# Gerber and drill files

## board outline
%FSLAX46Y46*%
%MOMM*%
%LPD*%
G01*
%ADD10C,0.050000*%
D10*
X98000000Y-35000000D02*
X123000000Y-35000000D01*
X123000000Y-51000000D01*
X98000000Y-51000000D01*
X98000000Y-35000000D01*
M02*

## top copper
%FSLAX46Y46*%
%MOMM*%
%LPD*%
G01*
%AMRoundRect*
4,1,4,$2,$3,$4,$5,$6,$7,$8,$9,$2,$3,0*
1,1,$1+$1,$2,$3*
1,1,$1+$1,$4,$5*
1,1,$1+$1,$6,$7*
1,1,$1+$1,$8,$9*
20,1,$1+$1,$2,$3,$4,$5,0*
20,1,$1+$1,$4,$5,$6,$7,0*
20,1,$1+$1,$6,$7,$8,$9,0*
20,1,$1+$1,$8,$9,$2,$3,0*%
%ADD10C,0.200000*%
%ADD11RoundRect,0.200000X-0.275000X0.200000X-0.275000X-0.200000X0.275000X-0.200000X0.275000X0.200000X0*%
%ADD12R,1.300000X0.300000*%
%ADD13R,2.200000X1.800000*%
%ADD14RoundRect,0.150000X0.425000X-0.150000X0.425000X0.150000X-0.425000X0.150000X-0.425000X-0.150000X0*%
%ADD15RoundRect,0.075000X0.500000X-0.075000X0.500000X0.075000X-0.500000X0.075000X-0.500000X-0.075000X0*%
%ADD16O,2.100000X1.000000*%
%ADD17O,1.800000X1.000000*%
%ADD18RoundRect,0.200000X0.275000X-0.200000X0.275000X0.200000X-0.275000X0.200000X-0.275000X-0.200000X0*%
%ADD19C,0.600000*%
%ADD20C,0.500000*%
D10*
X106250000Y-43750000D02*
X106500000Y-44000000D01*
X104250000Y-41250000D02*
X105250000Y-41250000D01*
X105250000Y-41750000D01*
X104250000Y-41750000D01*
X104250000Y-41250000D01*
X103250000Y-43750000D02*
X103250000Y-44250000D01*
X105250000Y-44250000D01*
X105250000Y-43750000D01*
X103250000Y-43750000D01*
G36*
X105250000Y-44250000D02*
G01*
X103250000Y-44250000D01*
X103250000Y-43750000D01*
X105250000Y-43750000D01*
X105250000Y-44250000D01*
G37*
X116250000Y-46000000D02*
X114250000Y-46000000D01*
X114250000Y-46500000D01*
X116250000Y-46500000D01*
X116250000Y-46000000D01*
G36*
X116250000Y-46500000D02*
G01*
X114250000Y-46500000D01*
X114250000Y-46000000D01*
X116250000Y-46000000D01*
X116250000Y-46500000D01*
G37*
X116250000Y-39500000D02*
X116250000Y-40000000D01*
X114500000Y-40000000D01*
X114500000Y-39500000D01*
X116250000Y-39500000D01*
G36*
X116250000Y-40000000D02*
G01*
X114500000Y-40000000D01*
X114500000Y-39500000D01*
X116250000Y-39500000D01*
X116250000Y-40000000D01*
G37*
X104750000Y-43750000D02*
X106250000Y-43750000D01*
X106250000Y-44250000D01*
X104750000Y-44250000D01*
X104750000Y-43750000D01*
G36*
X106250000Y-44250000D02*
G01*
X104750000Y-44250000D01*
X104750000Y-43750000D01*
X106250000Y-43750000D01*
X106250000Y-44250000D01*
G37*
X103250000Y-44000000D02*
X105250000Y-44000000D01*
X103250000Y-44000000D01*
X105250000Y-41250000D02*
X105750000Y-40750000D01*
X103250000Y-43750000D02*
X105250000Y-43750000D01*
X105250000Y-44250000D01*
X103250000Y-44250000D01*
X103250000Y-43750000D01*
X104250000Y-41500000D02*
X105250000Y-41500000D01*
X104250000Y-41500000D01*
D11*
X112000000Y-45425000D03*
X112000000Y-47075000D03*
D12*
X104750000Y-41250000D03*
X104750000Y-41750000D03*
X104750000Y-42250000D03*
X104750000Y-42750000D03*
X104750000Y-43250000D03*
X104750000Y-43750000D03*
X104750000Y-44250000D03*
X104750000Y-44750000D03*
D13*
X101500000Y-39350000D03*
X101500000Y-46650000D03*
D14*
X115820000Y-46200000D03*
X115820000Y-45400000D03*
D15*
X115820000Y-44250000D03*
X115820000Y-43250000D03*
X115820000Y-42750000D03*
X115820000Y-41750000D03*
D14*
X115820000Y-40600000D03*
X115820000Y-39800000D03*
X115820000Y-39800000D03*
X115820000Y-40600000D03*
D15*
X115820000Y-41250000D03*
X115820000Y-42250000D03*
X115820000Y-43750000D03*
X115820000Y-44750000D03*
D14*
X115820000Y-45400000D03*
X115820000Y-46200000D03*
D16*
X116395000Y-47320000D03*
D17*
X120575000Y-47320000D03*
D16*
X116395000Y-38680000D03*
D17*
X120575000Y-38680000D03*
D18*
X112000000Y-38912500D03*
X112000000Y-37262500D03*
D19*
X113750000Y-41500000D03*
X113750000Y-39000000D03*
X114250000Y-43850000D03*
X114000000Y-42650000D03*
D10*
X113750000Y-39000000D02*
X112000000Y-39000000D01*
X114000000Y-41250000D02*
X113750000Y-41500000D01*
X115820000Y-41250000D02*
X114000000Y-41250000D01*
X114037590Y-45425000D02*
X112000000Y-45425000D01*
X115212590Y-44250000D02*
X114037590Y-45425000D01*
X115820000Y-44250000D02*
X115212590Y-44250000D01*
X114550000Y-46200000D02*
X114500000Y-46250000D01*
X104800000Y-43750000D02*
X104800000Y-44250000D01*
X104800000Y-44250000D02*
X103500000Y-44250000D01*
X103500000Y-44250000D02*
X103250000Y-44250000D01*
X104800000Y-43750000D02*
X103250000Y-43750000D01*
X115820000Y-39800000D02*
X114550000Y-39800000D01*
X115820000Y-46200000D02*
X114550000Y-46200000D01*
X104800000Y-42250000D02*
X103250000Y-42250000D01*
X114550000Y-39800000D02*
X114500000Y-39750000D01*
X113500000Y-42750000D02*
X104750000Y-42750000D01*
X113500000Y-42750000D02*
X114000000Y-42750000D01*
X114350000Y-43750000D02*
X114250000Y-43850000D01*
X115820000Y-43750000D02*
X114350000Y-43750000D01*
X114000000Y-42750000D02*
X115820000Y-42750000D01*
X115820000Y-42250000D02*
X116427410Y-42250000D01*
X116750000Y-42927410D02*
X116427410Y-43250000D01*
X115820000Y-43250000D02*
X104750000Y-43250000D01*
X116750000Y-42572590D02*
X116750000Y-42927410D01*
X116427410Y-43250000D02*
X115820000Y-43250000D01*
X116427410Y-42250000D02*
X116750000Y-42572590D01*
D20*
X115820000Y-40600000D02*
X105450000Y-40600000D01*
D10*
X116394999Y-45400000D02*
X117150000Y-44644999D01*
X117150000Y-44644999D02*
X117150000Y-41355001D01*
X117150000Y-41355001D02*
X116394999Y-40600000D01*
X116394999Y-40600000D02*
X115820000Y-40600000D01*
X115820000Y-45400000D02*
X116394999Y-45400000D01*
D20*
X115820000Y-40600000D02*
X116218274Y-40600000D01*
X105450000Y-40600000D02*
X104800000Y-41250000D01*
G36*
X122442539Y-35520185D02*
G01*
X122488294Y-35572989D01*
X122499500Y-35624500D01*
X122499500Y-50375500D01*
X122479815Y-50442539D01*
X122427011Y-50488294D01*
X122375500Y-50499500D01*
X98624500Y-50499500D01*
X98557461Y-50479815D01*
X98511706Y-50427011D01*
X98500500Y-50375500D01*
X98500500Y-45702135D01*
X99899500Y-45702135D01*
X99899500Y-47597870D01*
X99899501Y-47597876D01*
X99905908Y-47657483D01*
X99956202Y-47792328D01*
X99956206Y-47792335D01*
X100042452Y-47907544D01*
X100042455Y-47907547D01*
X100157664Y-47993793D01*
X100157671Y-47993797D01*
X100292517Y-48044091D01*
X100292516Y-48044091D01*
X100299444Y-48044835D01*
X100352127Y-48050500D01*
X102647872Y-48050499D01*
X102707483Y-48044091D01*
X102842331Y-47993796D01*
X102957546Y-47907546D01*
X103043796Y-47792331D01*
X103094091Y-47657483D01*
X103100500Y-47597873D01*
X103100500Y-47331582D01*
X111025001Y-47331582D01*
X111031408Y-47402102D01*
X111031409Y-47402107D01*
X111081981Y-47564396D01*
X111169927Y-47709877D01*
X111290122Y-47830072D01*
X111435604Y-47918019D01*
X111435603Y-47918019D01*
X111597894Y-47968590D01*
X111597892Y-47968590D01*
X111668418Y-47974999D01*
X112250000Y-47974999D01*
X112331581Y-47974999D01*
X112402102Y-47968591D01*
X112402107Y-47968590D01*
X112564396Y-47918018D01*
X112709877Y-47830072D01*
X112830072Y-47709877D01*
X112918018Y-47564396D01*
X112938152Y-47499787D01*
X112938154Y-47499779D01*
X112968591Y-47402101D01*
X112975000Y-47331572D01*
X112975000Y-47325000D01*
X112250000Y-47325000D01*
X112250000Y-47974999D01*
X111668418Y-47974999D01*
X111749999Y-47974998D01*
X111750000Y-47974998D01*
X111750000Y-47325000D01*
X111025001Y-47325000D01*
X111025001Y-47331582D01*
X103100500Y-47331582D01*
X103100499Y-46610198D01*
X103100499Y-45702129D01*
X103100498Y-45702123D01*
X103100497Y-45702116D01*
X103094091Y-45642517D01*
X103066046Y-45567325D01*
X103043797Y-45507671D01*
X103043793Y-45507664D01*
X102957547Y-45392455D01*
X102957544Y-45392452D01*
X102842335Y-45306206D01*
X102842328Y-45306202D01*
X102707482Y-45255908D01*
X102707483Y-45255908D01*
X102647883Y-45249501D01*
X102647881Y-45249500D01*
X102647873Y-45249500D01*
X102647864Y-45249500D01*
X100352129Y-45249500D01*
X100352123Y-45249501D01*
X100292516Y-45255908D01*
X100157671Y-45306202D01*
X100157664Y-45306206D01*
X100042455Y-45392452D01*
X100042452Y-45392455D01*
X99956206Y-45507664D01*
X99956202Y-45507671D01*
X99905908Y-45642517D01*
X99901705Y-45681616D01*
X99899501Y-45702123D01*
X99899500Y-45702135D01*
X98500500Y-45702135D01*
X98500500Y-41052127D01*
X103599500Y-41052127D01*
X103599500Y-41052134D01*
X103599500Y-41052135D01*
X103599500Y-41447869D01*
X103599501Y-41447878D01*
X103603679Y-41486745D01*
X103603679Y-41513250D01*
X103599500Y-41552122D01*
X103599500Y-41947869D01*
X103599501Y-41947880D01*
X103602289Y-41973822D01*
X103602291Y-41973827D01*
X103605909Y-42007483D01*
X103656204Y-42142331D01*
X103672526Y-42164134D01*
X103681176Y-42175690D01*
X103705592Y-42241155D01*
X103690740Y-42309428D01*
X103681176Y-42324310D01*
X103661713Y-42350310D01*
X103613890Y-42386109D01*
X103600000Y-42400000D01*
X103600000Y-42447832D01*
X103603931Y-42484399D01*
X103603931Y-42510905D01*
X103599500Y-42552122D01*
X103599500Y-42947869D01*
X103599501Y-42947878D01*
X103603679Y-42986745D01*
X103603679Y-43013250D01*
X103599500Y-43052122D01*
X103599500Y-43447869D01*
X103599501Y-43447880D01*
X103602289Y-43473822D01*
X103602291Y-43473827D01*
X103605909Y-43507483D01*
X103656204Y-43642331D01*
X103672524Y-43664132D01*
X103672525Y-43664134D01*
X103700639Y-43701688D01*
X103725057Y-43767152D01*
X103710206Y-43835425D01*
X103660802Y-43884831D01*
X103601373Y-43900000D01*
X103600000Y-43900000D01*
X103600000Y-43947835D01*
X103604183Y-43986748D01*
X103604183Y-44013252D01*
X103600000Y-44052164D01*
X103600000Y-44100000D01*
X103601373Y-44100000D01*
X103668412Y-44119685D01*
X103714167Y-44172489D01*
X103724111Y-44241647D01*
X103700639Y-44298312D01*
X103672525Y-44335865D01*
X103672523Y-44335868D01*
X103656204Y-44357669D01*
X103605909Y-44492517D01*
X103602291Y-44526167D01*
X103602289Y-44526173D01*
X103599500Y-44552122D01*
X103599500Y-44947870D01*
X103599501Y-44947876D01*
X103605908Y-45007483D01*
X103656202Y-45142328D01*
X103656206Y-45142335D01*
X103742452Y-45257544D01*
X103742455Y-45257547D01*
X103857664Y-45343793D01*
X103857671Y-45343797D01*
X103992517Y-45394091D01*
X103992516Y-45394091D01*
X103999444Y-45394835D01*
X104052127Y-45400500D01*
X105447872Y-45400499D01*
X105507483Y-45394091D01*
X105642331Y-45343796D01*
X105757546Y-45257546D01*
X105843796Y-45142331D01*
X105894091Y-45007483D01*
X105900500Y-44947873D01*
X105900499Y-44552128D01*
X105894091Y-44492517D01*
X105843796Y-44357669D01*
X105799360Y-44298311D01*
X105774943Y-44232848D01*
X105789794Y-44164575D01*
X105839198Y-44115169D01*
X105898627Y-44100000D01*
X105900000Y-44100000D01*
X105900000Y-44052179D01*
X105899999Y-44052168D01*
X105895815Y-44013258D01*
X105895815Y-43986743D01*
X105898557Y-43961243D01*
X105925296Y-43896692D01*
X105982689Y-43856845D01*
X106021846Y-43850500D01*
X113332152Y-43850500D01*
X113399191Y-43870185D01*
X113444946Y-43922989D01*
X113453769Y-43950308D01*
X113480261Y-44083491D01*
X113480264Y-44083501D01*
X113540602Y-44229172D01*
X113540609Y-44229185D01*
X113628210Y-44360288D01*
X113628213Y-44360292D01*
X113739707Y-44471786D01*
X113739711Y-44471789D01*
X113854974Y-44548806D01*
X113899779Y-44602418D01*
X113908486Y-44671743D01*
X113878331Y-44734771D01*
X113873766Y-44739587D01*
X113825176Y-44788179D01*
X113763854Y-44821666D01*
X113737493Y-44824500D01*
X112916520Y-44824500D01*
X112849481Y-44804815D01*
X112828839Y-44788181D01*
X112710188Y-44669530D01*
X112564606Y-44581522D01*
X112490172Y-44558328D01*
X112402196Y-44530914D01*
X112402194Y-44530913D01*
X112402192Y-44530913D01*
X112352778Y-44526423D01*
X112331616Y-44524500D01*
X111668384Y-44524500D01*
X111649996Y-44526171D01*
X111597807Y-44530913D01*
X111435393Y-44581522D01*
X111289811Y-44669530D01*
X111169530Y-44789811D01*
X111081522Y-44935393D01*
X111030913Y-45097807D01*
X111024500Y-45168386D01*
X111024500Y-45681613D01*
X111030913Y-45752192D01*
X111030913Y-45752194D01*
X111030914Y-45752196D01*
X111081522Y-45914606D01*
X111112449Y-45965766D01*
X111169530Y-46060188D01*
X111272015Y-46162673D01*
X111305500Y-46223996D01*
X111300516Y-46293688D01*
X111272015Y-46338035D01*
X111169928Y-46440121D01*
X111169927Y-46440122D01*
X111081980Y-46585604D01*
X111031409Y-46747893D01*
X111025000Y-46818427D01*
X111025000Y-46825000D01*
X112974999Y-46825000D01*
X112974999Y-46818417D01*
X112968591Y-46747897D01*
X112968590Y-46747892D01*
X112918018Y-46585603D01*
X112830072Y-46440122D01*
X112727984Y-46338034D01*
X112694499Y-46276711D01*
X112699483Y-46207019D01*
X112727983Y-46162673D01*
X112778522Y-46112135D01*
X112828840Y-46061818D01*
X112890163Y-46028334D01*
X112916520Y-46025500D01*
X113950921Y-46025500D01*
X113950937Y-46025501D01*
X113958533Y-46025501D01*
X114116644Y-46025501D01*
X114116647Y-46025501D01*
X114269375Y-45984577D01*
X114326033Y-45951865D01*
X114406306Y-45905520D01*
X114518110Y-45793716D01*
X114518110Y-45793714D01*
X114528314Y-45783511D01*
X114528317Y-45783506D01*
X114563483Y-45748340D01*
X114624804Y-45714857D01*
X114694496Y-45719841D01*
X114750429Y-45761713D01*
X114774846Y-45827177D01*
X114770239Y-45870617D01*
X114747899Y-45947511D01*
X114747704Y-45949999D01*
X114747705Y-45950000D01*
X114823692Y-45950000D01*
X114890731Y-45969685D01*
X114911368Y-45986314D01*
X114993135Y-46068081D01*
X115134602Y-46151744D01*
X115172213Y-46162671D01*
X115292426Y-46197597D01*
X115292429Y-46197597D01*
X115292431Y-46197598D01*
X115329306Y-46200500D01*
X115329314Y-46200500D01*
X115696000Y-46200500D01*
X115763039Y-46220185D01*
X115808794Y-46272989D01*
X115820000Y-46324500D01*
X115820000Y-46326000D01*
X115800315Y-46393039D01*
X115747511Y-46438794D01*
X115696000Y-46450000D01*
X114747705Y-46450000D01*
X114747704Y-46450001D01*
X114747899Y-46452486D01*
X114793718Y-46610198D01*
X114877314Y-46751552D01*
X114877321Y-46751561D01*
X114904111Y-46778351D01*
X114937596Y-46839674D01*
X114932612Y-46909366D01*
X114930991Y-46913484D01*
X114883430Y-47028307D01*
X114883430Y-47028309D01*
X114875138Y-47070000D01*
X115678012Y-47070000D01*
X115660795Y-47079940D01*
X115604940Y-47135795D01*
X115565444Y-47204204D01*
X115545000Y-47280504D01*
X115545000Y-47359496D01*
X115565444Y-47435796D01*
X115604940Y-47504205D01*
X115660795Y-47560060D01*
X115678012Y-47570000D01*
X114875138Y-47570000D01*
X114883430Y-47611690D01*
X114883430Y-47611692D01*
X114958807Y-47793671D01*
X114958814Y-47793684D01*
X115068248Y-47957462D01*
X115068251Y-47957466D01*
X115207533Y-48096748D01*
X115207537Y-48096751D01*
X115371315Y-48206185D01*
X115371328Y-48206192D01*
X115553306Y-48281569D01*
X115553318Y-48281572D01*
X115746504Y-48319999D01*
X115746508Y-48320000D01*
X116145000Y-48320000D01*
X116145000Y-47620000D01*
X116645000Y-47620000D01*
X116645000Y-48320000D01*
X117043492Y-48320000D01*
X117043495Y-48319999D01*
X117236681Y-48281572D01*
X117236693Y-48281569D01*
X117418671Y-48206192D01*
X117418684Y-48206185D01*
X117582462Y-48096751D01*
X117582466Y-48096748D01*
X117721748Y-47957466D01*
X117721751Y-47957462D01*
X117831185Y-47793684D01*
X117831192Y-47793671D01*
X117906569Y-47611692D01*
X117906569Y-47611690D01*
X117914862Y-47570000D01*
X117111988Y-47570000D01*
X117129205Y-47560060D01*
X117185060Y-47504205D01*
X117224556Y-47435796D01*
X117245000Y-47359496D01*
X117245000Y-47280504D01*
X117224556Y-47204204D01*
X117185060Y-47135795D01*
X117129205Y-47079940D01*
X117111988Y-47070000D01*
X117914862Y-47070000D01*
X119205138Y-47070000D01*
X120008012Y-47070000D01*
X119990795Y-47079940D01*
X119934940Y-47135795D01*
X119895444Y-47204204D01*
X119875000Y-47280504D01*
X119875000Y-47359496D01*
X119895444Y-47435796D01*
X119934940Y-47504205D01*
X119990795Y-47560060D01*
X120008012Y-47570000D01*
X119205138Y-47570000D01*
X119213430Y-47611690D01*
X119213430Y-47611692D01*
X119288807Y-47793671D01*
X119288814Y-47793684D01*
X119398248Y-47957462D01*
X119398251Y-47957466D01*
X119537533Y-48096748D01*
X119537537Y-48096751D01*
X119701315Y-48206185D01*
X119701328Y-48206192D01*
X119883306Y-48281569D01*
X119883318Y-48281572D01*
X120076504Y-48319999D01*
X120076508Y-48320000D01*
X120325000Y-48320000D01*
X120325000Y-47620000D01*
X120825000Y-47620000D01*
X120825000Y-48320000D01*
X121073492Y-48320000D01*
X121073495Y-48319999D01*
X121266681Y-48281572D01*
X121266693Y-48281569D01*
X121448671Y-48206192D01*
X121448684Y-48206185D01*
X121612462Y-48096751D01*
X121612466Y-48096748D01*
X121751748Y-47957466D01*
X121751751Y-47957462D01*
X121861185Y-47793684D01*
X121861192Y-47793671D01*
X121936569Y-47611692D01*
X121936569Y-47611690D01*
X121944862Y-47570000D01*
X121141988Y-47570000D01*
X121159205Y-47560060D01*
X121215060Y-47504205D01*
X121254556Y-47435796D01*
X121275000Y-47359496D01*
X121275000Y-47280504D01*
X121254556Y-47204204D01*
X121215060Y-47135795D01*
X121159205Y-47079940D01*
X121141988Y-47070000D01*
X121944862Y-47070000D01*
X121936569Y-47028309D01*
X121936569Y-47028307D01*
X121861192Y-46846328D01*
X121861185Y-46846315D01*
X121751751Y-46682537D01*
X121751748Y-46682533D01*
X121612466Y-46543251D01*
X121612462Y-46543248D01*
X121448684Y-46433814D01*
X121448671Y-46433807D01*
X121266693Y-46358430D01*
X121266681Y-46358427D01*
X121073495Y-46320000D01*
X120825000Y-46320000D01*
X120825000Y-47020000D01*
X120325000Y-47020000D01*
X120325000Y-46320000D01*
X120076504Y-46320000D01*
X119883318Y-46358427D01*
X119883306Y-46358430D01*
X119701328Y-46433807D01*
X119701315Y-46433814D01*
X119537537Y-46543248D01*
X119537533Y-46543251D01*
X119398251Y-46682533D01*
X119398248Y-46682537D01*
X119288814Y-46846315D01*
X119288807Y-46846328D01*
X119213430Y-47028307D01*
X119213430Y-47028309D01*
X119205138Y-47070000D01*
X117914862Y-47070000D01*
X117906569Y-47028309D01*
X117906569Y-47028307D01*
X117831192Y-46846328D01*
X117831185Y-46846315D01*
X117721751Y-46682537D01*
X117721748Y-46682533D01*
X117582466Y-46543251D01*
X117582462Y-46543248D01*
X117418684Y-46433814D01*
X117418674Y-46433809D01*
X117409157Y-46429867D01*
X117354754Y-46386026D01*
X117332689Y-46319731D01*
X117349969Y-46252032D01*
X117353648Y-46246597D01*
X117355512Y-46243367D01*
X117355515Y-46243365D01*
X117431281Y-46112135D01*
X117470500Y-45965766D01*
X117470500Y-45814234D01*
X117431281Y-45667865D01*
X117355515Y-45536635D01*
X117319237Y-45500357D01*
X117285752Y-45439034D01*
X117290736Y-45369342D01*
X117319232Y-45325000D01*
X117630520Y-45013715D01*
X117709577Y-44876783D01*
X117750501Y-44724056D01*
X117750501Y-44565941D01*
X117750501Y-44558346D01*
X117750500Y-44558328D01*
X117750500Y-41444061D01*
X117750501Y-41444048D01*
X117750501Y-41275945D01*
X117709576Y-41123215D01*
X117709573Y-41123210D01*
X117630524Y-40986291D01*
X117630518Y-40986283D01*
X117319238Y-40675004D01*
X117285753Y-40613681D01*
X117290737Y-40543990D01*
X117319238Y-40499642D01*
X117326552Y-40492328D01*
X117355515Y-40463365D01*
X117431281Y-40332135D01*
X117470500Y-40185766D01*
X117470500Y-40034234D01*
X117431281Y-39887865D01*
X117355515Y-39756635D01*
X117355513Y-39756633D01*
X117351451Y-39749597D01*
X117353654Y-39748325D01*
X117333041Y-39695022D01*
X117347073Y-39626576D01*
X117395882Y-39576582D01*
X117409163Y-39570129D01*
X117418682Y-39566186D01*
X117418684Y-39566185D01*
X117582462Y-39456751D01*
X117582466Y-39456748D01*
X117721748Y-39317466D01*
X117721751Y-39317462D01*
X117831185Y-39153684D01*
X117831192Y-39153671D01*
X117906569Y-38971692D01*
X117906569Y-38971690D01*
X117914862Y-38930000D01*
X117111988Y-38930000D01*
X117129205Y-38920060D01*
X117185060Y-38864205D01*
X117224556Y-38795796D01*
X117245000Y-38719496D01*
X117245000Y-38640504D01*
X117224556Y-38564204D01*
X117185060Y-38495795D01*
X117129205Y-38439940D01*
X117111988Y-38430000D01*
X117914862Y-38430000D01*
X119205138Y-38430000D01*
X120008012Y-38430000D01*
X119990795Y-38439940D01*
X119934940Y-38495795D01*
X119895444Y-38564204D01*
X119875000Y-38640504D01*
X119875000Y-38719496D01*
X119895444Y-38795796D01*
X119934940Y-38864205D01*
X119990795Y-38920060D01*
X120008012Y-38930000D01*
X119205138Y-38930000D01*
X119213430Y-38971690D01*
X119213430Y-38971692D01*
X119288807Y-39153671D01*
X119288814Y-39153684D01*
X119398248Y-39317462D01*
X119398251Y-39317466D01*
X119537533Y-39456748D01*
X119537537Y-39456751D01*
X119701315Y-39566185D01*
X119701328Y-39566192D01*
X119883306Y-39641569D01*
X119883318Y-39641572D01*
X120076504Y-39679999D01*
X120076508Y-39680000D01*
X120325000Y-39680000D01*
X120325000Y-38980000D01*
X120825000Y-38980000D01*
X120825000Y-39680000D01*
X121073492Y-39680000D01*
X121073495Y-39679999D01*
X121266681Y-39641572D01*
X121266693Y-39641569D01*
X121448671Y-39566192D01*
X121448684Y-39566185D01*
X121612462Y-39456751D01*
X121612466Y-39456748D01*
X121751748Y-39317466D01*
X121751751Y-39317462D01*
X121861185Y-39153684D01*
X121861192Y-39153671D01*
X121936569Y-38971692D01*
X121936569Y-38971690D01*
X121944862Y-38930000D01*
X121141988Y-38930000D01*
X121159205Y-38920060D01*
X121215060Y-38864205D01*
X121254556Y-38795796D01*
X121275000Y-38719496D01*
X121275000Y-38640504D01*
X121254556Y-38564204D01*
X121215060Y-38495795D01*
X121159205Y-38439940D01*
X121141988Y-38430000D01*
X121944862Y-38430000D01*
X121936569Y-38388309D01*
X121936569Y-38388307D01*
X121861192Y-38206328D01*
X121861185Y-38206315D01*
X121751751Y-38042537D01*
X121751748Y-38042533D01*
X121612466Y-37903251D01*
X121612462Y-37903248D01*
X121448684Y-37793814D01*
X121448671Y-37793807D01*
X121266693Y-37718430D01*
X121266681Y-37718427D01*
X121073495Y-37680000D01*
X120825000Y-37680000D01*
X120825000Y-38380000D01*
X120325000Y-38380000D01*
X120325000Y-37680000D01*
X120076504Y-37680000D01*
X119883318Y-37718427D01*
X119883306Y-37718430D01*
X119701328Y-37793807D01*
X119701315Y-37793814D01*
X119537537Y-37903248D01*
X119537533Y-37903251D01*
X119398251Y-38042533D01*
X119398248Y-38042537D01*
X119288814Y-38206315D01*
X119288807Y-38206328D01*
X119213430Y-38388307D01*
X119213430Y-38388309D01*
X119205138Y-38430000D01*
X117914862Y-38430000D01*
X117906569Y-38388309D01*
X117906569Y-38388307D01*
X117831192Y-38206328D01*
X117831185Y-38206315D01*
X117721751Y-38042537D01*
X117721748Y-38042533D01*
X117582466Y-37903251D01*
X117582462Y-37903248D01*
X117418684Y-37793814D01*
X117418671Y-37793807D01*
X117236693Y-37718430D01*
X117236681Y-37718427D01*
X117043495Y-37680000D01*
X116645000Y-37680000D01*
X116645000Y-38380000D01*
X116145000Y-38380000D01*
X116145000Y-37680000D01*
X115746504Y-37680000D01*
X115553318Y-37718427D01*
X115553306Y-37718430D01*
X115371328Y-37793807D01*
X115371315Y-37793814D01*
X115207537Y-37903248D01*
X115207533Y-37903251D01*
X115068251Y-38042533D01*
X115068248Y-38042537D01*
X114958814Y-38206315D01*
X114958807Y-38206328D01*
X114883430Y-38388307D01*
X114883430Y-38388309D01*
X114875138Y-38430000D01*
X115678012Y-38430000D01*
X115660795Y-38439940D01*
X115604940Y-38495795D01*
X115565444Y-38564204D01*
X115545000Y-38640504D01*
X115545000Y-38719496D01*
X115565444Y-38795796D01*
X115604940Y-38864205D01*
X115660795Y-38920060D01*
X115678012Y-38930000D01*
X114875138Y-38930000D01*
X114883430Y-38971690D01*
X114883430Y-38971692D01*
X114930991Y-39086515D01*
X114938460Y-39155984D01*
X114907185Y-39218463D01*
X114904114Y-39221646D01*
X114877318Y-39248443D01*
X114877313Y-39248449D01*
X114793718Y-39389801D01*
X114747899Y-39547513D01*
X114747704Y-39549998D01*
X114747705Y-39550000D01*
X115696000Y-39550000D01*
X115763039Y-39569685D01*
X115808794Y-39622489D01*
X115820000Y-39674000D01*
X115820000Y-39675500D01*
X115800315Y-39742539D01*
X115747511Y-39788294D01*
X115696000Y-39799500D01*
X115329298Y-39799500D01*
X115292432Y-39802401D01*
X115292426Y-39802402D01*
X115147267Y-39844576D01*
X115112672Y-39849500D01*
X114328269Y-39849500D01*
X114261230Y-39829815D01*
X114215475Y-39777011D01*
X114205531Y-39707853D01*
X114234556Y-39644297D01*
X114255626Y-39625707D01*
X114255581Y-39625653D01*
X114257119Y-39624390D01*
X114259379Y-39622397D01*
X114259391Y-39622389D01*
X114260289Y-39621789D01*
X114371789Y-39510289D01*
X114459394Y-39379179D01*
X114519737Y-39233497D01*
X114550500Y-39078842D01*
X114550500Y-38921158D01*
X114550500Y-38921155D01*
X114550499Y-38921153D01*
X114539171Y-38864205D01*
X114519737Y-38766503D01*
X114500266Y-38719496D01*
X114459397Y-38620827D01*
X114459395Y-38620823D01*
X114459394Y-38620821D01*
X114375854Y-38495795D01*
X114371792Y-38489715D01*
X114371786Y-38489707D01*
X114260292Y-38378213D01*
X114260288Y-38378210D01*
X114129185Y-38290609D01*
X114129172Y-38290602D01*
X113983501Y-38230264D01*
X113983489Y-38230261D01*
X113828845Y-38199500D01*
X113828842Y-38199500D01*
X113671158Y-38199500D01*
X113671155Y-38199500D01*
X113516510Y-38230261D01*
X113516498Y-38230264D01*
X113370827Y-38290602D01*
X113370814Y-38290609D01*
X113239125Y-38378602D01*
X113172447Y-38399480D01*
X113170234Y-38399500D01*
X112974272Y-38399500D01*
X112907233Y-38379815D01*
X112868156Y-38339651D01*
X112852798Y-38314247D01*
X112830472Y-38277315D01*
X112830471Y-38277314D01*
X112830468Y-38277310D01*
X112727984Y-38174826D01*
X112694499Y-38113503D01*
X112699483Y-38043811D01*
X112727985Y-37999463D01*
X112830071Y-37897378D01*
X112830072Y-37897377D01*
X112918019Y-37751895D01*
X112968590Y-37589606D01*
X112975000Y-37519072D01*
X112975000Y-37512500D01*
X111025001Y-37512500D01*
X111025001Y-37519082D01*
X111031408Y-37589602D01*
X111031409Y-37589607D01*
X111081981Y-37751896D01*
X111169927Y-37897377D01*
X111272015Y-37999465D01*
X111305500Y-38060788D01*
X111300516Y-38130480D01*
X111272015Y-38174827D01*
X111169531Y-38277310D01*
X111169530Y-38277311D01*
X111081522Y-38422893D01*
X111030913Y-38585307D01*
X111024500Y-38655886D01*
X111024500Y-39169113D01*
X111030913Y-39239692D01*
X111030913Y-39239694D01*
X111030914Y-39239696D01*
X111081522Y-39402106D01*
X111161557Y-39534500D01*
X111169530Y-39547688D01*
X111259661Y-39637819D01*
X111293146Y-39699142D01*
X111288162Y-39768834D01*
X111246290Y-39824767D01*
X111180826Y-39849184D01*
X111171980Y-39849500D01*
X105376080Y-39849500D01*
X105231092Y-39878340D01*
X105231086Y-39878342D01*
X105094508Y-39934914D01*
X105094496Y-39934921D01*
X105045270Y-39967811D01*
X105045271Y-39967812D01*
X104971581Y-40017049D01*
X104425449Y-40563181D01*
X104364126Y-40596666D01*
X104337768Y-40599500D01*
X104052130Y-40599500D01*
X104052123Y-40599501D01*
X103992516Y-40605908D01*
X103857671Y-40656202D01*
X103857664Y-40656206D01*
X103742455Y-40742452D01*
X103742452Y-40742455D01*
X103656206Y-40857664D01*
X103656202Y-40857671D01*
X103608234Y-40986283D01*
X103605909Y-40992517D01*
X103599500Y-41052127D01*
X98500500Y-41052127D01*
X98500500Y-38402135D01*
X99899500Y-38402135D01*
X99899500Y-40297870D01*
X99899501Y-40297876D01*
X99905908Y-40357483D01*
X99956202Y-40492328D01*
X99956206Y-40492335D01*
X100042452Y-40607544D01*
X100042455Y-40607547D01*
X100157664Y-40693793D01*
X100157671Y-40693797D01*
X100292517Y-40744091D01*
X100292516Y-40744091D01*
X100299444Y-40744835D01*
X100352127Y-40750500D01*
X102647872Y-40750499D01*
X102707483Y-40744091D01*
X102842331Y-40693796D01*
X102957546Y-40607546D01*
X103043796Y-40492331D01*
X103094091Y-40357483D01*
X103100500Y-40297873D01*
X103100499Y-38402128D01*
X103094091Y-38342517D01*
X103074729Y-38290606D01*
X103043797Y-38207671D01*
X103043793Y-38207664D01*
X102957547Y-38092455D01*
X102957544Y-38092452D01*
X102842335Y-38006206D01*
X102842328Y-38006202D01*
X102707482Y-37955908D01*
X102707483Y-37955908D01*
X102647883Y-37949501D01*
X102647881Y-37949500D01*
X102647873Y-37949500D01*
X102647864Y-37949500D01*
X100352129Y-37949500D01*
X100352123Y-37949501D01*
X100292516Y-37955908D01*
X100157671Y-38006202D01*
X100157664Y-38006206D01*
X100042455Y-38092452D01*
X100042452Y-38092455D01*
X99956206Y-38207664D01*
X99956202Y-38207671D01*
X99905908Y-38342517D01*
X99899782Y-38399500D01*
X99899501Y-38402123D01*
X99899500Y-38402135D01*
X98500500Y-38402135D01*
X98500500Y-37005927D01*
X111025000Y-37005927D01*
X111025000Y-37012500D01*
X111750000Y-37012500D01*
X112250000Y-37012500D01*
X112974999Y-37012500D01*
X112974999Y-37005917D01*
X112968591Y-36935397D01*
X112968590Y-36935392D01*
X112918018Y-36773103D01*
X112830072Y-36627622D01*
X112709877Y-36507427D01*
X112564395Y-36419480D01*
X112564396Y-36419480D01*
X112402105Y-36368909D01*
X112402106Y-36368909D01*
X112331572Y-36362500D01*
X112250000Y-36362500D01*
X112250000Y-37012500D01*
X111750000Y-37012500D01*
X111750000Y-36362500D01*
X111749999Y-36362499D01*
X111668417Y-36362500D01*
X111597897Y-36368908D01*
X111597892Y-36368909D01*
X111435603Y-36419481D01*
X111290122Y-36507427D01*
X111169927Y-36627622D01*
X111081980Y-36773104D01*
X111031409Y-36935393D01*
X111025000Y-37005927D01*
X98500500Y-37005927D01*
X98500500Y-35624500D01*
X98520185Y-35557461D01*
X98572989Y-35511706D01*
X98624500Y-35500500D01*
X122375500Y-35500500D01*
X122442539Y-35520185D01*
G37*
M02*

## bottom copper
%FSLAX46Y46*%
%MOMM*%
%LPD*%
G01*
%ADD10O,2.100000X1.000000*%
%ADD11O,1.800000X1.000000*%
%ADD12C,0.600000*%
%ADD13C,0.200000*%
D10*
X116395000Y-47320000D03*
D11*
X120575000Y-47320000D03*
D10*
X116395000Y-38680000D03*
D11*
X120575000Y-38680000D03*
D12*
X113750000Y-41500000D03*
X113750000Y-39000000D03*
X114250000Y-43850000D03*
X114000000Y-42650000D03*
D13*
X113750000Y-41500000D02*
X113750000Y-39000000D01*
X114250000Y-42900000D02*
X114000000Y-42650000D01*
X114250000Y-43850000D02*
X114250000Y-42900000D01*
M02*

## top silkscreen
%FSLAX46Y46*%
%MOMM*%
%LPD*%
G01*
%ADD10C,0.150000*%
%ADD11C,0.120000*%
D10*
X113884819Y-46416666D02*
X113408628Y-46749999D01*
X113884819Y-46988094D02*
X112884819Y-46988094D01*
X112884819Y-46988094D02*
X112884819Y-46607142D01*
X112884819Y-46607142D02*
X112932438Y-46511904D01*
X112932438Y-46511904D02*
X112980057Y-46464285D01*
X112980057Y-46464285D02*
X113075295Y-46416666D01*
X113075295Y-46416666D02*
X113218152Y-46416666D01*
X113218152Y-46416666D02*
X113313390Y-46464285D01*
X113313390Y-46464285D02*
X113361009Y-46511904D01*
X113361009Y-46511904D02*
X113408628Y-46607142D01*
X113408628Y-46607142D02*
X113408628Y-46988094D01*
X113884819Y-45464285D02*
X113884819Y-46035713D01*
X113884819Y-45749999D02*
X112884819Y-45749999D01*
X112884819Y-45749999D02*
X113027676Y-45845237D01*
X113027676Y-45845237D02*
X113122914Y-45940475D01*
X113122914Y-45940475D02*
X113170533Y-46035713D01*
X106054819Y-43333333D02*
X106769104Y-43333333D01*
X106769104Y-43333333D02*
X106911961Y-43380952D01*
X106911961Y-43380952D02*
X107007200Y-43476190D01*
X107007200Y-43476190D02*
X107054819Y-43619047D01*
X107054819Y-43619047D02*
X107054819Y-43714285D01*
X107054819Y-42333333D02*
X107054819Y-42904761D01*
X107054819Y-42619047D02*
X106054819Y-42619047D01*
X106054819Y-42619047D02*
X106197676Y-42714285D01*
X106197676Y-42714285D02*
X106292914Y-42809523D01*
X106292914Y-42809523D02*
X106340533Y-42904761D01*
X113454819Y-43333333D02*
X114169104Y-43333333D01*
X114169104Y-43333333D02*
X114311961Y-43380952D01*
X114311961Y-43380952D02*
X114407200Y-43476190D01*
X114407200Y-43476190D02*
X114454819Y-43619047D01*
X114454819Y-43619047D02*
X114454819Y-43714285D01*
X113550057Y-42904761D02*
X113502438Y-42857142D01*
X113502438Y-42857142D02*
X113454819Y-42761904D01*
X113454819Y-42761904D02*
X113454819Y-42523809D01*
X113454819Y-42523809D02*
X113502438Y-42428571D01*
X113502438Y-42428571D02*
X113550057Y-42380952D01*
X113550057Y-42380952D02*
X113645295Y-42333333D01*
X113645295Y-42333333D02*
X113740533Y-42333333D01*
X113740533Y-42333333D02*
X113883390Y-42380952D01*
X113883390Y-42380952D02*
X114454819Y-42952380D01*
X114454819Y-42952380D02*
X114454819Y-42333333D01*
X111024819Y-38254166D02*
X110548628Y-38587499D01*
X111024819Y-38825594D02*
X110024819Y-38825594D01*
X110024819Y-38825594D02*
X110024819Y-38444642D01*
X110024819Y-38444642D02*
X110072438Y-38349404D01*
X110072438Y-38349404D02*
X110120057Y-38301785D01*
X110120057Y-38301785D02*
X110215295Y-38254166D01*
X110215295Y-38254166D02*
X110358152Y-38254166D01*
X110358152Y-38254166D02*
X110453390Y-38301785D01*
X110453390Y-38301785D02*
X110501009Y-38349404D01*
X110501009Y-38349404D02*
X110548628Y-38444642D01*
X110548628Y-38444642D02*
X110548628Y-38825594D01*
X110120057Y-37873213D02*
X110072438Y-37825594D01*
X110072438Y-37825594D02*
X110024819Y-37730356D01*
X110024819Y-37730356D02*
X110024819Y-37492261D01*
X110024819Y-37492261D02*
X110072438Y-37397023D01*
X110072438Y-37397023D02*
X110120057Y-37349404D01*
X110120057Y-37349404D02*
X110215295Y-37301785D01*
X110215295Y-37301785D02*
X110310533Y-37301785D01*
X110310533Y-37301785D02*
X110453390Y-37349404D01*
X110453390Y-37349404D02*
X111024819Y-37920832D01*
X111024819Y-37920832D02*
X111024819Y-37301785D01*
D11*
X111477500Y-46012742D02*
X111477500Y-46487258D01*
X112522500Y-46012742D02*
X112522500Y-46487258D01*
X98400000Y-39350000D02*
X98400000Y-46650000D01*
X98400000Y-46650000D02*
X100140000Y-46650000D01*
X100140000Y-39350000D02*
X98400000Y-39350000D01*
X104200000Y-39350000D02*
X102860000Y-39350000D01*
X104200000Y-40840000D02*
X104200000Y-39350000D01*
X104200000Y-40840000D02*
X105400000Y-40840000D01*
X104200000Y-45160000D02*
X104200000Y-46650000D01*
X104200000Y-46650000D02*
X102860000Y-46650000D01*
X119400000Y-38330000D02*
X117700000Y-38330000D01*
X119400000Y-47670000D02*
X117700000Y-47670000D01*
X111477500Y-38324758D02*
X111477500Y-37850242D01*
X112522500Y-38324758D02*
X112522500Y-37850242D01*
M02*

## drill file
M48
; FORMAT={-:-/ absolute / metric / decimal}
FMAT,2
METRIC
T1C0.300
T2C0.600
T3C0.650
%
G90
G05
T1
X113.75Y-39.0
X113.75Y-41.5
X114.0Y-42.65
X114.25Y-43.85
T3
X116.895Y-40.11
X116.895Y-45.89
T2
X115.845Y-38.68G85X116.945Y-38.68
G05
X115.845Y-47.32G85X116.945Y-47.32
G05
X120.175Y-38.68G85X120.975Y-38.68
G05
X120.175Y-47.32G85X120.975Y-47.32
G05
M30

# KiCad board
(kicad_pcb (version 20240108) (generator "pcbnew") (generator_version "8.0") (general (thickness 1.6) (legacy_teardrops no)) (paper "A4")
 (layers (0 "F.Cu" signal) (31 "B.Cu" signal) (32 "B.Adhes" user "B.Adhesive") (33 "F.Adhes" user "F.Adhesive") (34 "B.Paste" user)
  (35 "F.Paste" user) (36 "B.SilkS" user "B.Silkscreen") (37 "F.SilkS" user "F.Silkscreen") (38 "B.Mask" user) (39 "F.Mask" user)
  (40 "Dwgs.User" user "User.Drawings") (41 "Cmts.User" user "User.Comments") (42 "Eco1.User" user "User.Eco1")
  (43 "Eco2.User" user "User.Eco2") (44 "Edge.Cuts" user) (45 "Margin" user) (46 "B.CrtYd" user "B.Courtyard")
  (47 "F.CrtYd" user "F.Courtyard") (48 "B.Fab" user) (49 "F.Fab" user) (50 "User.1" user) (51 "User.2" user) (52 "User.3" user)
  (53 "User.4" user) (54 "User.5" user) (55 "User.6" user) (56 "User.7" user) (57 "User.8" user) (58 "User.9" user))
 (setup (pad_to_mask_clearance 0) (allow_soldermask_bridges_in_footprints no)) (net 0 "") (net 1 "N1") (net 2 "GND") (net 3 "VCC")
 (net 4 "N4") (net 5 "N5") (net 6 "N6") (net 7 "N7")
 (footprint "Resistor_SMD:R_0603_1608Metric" (layer "F.Cu") (at 112 46.25 -90)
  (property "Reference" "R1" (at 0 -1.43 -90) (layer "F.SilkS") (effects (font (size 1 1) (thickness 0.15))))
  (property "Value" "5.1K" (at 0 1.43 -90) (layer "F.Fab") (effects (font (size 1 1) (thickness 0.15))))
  (fp_line (start -0.237258 0.5225) (end 0.237258 0.5225) (stroke (width 0.12) (type solid)) (layer "F.SilkS"))
  (fp_line (start -0.237258 -0.5225) (end 0.237258 -0.5225) (stroke (width 0.12) (type solid)) (layer "F.SilkS"))
  (pad "1" smd roundrect (at -0.825 0 270) (size 0.8 0.95) (layers "F.Cu" "F.Paste" "F.Mask") (roundrect_rratio 0.25) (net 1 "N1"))
  (pad "2" smd roundrect (at 0.825 0 270) (size 0.8 0.95) (layers "F.Cu" "F.Paste" "F.Mask") (roundrect_rratio 0.25) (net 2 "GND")))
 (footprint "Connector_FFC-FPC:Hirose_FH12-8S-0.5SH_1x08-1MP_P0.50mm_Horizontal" (layer "F.Cu") (at 102.9 43 -90)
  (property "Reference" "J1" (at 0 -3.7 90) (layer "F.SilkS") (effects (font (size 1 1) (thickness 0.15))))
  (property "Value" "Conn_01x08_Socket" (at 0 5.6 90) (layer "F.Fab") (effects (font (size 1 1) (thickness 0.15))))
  (fp_line (start -3.65 4.5) (end 3.65 4.5) (stroke (width 0.12) (type solid)) (layer "F.SilkS"))
  (fp_line (start 3.65 4.5) (end 3.65 2.76) (stroke (width 0.12) (type solid)) (layer "F.SilkS"))
  (fp_line (start -3.65 2.76) (end -3.65 4.5) (stroke (width 0.12) (type solid)) (layer "F.SilkS"))
  (fp_line (start -3.65 -1.3) (end -3.65 0.04) (stroke (width 0.12) (type solid)) (layer "F.SilkS"))
  (fp_line (start -2.16 -1.3) (end -3.65 -1.3) (stroke (width 0.12) (type solid)) (layer "F.SilkS"))
  (fp_line (start -2.16 -1.3) (end -2.16 -2.5) (stroke (width 0.12) (type solid)) (layer "F.SilkS"))
  (fp_line (start 2.16 -1.3) (end 3.65 -1.3) (stroke (width 0.12) (type solid)) (layer "F.SilkS"))
  (fp_line (start 3.65 -1.3) (end 3.65 0.04) (stroke (width 0.12) (type solid)) (layer "F.SilkS"))
  (pad "1" smd rect (at -1.75 -1.85 270) (size 0.3 1.3) (layers "F.Cu" "F.Paste" "F.Mask") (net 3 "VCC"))
  (pad "2" smd rect (at -1.25 -1.85 270) (size 0.3 1.3) (layers "F.Cu" "F.Paste" "F.Mask") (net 3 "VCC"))
  (pad "3" smd rect (at -0.75 -1.85 270) (size 0.3 1.3) (layers "F.Cu" "F.Paste" "F.Mask") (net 2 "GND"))
  (pad "4" smd rect (at -0.25 -1.85 270) (size 0.3 1.3) (layers "F.Cu" "F.Paste" "F.Mask") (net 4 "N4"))
  (pad "5" smd rect (at 0.25 -1.85 270) (size 0.3 1.3) (layers "F.Cu" "F.Paste" "F.Mask") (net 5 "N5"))
  (pad "6" smd rect (at 0.75 -1.85 270) (size 0.3 1.3) (layers "F.Cu" "F.Paste" "F.Mask") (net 2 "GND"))
  (pad "7" smd rect (at 1.25 -1.85 270) (size 0.3 1.3) (layers "F.Cu" "F.Paste" "F.Mask") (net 2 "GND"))
  (pad "8" smd rect (at 1.75 -1.85 270) (size 0.3 1.3) (layers "F.Cu" "F.Paste" "F.Mask") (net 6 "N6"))
  (pad "MP" smd rect (at -3.65 1.4 270) (size 1.8 2.2) (layers "F.Cu" "F.Paste" "F.Mask"))
  (pad "MP" smd rect (at 3.65 1.4 270) (size 1.8 2.2) (layers "F.Cu" "F.Paste" "F.Mask")))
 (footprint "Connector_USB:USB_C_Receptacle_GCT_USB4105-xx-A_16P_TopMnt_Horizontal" (layer "F.Cu") (at 119.5 43 90)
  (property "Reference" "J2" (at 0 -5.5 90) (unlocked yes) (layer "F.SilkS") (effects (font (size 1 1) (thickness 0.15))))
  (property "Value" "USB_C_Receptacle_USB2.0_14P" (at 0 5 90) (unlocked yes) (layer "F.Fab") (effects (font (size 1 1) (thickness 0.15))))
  (fp_line (start 4.67 -0.1) (end 4.67 -1.8) (stroke (width 0.12) (type solid)) (layer "F.SilkS"))
  (fp_line (start -4.67 -0.1) (end -4.67 -1.8) (stroke (width 0.12) (type solid)) (layer "F.SilkS"))
  (pad "" np_thru_hole circle (at -2.89 -2.605 90) (size 0.65 0.65) (drill 0.65) (layers "F&B.Cu" "*.Mask"))
  (pad "" np_thru_hole circle (at 2.89 -2.605 90) (size 0.65 0.65) (drill 0.65) (layers "F&B.Cu" "*.Mask"))
  (pad "A1" smd roundrect (at -3.2 -3.68 90) (size 0.6 1.15) (layers "F.Cu" "F.Paste" "F.Mask") (roundrect_rratio 0.25) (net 2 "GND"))
  (pad "A4" smd roundrect (at -2.4 -3.68 90) (size 0.6 1.15) (layers "F.Cu" "F.Paste" "F.Mask") (roundrect_rratio 0.25) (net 3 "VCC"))
  (pad "A5" smd roundrect (at -1.25 -3.68 90) (size 0.3 1.15) (layers "F.Cu" "F.Paste" "F.Mask") (roundrect_rratio 0.25) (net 1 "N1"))
  (pad "A6" smd roundrect (at -0.25 -3.68 90) (size 0.3 1.15) (layers "F.Cu" "F.Paste" "F.Mask") (roundrect_rratio 0.25) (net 5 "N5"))
  (pad "A7" smd roundrect (at 0.25 -3.68 90) (size 0.3 1.15) (layers "F.Cu" "F.Paste" "F.Mask") (roundrect_rratio 0.25) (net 4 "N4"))
  (pad "A8" smd roundrect (at 1.25 -3.68 90) (size 0.3 1.15) (layers "F.Cu" "F.Paste" "F.Mask") (roundrect_rratio 0.25))
  (pad "A9" smd roundrect (at 2.4 -3.68 90) (size 0.6 1.15) (layers "F.Cu" "F.Paste" "F.Mask") (roundrect_rratio 0.25) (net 3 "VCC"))
  (pad "A12" smd roundrect (at 3.2 -3.68 90) (size 0.6 1.15) (layers "F.Cu" "F.Paste" "F.Mask") (roundrect_rratio 0.25) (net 2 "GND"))
  (pad "B1" smd roundrect (at 3.2 -3.68 90) (size 0.6 1.15) (layers "F.Cu" "F.Paste" "F.Mask") (roundrect_rratio 0.25) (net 2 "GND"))
  (pad "B4" smd roundrect (at 2.4 -3.68 90) (size 0.6 1.15) (layers "F.Cu" "F.Paste" "F.Mask") (roundrect_rratio 0.25) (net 3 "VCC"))
  (pad "B5" smd roundrect (at 1.75 -3.68 90) (size 0.3 1.15) (layers "F.Cu" "F.Paste" "F.Mask") (roundrect_rratio 0.25) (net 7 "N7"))
  (pad "B6" smd roundrect (at 0.75 -3.68 90) (size 0.3 1.15) (layers "F.Cu" "F.Paste" "F.Mask") (roundrect_rratio 0.25) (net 5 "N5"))
  (pad "B7" smd roundrect (at -0.75 -3.68 90) (size 0.3 1.15) (layers "F.Cu" "F.Paste" "F.Mask") (roundrect_rratio 0.25) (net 4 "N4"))
  (pad "B8" smd roundrect (at -1.75 -3.68 90) (size 0.3 1.15) (layers "F.Cu" "F.Paste" "F.Mask") (roundrect_rratio 0.25))
  (pad "B9" smd roundrect (at -2.4 -3.68 90) (size 0.6 1.15) (layers "F.Cu" "F.Paste" "F.Mask") (roundrect_rratio 0.25) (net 3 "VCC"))
  (pad "B12" smd roundrect (at -3.2 -3.68 90) (size 0.6 1.15) (layers "F.Cu" "F.Paste" "F.Mask") (roundrect_rratio 0.25) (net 2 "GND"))
  (pad "S1" thru_hole oval (at -4.32 -3.105 90) (size 1 2.1) (drill oval 0.6 1.7) (layers "*.Cu" "*.Mask" "F.Paste")
   (remove_unused_layers no) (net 2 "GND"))
  (pad "S1" thru_hole oval (at -4.32 1.075 90) (size 1 1.8) (drill oval 0.6 1.4) (layers "*.Cu" "*.Mask" "F.Paste")
   (remove_unused_layers no) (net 2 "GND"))
  (pad "S1" thru_hole oval (at 4.32 -3.105 90) (size 1 2.1) (drill oval 0.6 1.7) (layers "*.Cu" "*.Mask" "F.Paste")
   (remove_unused_layers no) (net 2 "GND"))
  (pad "S1" thru_hole oval (at 4.32 1.075 90) (size 1 1.8) (drill oval 0.6 1.4) (layers "*.Cu" "*.Mask" "F.Paste") (remove_unused_layers no)
   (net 2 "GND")))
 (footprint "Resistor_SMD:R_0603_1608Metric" (layer "F.Cu") (at 112 38.0875 90)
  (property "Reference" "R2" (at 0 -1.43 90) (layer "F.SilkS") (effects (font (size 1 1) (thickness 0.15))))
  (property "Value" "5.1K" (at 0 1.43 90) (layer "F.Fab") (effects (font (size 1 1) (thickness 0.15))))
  (fp_line (start -0.237258 -0.5225) (end 0.237258 -0.5225) (stroke (width 0.12) (type solid)) (layer "F.SilkS"))
  (fp_line (start -0.237258 0.5225) (end 0.237258 0.5225) (stroke (width 0.12) (type solid)) (layer "F.SilkS"))
  (pad "1" smd roundrect (at -0.825 0 90) (size 0.8 0.95) (layers "F.Cu" "F.Paste" "F.Mask") (roundrect_rratio 0.25) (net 7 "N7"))
  (pad "2" smd roundrect (at 0.825 0 90) (size 0.8 0.95) (layers "F.Cu" "F.Paste" "F.Mask") (roundrect_rratio 0.25) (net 2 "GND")))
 (gr_line (start 106.25 43.75) (end 106.5 44) (stroke (width 0.2) (type default)) (layer "F.Cu") (net 2))
 (gr_rect (start 104.25 41.25) (end 105.25 41.75) (stroke (width 0.2) (type default)) (fill none) (layer "F.Cu") (net 3))
 (gr_poly
  (pts (xy 103.25 43.75) (xy 103.25 44.25) (xy 105.25 44.25) (xy 105.25 43.75)) (stroke (width 0.2) (type solid)) (fill solid)
  (layer "F.Cu") (net 2))
 (gr_poly
  (pts (xy 116.25 46) (xy 114.25 46) (xy 114.25 46.5) (xy 116.25 46.5)) (stroke (width 0.2) (type solid)) (fill solid) (layer "F.Cu")
  (net 2))
 (gr_poly
  (pts (xy 116.25 39.5) (xy 116.25 40) (xy 114.5 40) (xy 114.5 39.5)) (stroke (width 0.2) (type solid)) (fill solid) (layer "F.Cu") (net 2))
 (gr_poly
  (pts (xy 104.75 43.75) (xy 106.25 43.75) (xy 106.25 44.25) (xy 104.75 44.25)) (stroke (width 0.2) (type solid)) (fill solid)
  (layer "F.Cu") (net 2))
 (gr_rect (start 103.25 44) (end 105.25 44) (stroke (width 0.2) (type default)) (fill none) (layer "F.Cu") (net 2))
 (gr_line (start 105.25 41.25) (end 105.75 40.75) (stroke (width 0.2) (type default)) (layer "F.Cu") (net 3))
 (gr_rect (start 103.25 43.75) (end 105.25 44.25) (stroke (width 0.2) (type default)) (fill none) (layer "F.Cu") (net 2))
 (gr_rect (start 104.25 41.5) (end 105.25 41.5) (stroke (width 0.2) (type default)) (fill none) (layer "F.Cu") (net 3))
 (gr_rect (start 98 35) (end 123 51) (stroke (width 0.05) (type default)) (fill none) (layer "Edge.Cuts"))
 (segment (start 113.75 39) (end 112 39) (width 0.2) (layer "F.Cu") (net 7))
 (segment (start 114 41.25) (end 113.75 41.5) (width 0.2) (layer "F.Cu") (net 7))
 (segment (start 115.82 41.25) (end 114 41.25) (width 0.2) (layer "F.Cu") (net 7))
 (via (at 113.75 41.5) (size 0.6) (drill 0.3) (layers "F.Cu" "B.Cu") (free yes) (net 7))
 (via (at 113.75 39) (size 0.6) (drill 0.3) (layers "F.Cu" "B.Cu") (free yes) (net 7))
 (segment (start 113.75 41.5) (end 113.75 39) (width 0.2) (layer "B.Cu") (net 7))
 (segment (start 114.03759 45.425) (end 112 45.425) (width 0.2) (layer "F.Cu") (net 1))
 (segment (start 115.21259 44.25) (end 114.03759 45.425) (width 0.2) (layer "F.Cu") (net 1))
 (segment (start 115.82 44.25) (end 115.21259 44.25) (width 0.2) (layer "F.Cu") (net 1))
 (segment (start 114.55 46.2) (end 114.5 46.25) (width 0.2) (layer "F.Cu") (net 2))
 (segment (start 104.8 43.75) (end 104.8 44.25) (width 0.2) (layer "F.Cu") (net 2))
 (segment (start 104.8 44.25) (end 103.5 44.25) (width 0.2) (layer "F.Cu") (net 2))
 (segment (start 103.5 44.25) (end 103.25 44.25) (width 0.2) (layer "F.Cu") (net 2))
 (segment (start 104.8 43.75) (end 103.25 43.75) (width 0.2) (layer "F.Cu") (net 2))
 (segment (start 115.82 39.8) (end 114.55 39.8) (width 0.2) (layer "F.Cu") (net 2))
 (segment (start 115.82 46.2) (end 114.55 46.2) (width 0.2) (layer "F.Cu") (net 2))
 (segment (start 104.8 42.25) (end 103.25 42.25) (width 0.2) (layer "F.Cu") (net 2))
 (segment (start 114.55 39.8) (end 114.5 39.75) (width 0.2) (layer "F.Cu") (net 2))
 (segment (start 113.5 42.75) (end 104.75 42.75) (width 0.2) (layer "F.Cu") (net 4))
 (segment (start 113.5 42.75) (end 114 42.75) (width 0.2) (layer "F.Cu") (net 4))
 (segment (start 114.35 43.75) (end 114.25 43.85) (width 0.2) (layer "F.Cu") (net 4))
 (segment (start 115.82 43.75) (end 114.35 43.75) (width 0.2) (layer "F.Cu") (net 4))
 (segment (start 114 42.75) (end 115.82 42.75) (width 0.2) (layer "F.Cu") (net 4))
 (via (at 114.25 43.85) (size 0.6) (drill 0.3) (layers "F.Cu" "B.Cu") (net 4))
 (via (at 114 42.65) (size 0.6) (drill 0.3) (layers "F.Cu" "B.Cu") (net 4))
 (segment (start 114.25 42.9) (end 114 42.65) (width 0.2) (layer "B.Cu") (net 4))
 (segment (start 114.25 43.85) (end 114.25 42.9) (width 0.2) (layer "B.Cu") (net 4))
 (segment (start 115.82 42.25) (end 116.42741 42.25) (width 0.2) (layer "F.Cu") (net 5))
 (segment (start 116.75 42.92741) (end 116.42741 43.25) (width 0.2) (layer "F.Cu") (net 5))
 (segment (start 115.82 43.25) (end 104.75 43.25) (width 0.2) (layer "F.Cu") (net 5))
 (segment (start 116.75 42.57259) (end 116.75 42.92741) (width 0.2) (layer "F.Cu") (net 5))
 (segment (start 116.42741 43.25) (end 115.82 43.25) (width 0.2) (layer "F.Cu") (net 5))
 (segment (start 116.42741 42.25) (end 116.75 42.57259) (width 0.2) (layer "F.Cu") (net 5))
 (segment (start 115.82 40.6) (end 105.45 40.6) (width 0.5) (layer "F.Cu") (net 3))
 (segment (start 116.394999 45.4) (end 117.15 44.644999) (width 0.2) (layer "F.Cu") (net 3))
 (segment (start 117.15 44.644999) (end 117.15 41.355001) (width 0.2) (layer "F.Cu") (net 3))
 (segment (start 117.15 41.355001) (end 116.394999 40.6) (width 0.2) (layer "F.Cu") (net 3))
 (segment (start 116.394999 40.6) (end 115.82 40.6) (width 0.2) (layer "F.Cu") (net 3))
 (segment (start 115.82 45.4) (end 116.394999 45.4) (width 0.2) (layer "F.Cu") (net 3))
 (segment (start 115.82 40.6) (end 116.218274 40.6) (width 0.5) (layer "F.Cu") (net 3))
 (segment (start 105.45 40.6) (end 104.8 41.25) (width 0.5) (layer "F.Cu") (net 3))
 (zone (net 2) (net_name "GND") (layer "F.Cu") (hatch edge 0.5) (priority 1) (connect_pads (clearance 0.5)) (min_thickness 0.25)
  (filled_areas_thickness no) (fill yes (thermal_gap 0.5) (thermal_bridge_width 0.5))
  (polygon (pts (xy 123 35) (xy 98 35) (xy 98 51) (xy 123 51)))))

